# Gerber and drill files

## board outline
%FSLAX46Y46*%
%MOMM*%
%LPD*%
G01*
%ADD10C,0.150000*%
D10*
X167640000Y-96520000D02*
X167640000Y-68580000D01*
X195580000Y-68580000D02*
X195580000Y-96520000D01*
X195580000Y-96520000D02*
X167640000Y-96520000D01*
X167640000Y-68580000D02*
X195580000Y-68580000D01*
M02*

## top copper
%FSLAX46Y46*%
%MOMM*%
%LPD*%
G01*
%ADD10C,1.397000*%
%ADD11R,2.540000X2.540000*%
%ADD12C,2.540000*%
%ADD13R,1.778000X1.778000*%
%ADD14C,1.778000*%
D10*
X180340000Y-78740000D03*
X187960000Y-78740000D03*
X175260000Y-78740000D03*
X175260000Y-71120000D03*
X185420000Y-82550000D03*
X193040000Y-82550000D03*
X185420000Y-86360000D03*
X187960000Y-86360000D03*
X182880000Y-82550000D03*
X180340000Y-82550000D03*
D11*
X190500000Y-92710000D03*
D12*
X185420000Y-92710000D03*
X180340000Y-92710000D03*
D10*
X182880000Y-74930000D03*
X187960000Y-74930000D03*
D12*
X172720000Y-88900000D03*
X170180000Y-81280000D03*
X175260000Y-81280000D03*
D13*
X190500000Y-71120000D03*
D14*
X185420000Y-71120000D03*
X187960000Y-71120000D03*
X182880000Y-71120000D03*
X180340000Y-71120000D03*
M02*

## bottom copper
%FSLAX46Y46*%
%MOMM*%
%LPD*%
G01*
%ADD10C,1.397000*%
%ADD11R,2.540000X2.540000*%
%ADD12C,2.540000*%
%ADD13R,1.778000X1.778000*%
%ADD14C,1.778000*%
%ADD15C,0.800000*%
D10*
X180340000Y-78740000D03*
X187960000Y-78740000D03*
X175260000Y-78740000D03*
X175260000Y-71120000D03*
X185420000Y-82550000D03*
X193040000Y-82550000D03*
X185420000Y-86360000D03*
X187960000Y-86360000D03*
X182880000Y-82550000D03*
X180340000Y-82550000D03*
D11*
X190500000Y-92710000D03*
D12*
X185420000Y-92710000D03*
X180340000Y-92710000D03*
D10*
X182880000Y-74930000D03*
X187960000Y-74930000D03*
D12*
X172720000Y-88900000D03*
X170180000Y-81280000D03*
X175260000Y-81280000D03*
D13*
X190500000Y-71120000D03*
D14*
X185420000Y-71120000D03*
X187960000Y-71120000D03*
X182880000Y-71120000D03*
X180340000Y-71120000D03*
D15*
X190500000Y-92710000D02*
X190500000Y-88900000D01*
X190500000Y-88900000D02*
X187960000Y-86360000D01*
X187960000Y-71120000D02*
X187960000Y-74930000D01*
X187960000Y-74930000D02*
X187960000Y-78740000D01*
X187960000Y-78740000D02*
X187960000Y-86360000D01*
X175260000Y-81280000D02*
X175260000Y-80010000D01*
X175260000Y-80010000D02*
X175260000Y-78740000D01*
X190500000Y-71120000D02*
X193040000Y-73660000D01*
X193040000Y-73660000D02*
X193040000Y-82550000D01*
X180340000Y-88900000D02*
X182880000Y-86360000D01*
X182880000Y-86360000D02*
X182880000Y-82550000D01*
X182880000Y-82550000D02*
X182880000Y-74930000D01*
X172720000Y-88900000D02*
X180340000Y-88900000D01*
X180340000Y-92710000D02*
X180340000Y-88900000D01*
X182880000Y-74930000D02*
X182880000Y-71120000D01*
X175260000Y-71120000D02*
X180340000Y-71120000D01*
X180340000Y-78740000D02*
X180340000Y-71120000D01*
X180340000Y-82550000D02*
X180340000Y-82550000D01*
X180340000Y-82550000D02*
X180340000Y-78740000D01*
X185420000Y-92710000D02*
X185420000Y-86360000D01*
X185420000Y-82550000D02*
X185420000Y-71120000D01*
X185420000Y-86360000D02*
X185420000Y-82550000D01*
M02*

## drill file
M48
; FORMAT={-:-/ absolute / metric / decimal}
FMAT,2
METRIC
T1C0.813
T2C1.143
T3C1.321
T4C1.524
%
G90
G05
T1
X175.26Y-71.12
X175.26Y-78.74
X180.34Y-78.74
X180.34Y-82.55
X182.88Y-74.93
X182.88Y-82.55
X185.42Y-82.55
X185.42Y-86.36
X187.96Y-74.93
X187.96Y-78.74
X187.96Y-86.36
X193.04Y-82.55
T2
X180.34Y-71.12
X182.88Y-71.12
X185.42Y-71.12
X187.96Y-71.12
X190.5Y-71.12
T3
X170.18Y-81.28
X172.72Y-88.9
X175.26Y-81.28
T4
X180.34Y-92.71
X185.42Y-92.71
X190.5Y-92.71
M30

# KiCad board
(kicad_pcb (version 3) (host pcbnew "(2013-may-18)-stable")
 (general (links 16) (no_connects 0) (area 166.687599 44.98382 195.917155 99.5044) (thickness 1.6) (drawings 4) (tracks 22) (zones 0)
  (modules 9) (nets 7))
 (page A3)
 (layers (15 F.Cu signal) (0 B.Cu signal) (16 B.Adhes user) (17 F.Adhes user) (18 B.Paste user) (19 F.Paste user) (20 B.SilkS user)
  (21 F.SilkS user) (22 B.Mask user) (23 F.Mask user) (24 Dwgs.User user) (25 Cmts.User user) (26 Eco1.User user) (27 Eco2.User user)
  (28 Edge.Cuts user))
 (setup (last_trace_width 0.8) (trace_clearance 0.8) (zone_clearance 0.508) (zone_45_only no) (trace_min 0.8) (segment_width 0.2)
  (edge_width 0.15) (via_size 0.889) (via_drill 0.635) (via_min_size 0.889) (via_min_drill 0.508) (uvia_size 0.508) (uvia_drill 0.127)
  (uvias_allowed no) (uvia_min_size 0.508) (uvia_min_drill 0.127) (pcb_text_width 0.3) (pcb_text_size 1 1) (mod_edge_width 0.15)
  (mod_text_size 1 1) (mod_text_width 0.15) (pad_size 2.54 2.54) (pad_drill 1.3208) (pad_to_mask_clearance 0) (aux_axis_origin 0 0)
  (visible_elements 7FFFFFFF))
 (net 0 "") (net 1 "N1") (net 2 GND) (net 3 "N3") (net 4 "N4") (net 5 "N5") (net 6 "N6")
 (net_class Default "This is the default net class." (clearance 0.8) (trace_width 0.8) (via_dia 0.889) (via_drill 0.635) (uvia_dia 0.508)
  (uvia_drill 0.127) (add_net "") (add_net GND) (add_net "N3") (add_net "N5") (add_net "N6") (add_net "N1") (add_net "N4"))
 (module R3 (layer F.Cu) (at 184.15 78.74) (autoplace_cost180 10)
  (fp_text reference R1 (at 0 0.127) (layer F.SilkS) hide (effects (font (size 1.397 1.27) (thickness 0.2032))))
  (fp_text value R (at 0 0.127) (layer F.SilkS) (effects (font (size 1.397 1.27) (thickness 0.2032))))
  (pad 1 thru_hole circle (at -3.81 0) (size 1.397 1.397) (drill 0.8128) (layers *.Cu *.Mask F.SilkS) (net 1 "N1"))
  (pad 2 thru_hole circle (at 3.81 0) (size 1.397 1.397) (drill 0.8128) (layers *.Cu *.Mask F.SilkS) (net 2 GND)))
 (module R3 (layer F.Cu) (at 175.26 74.93 90) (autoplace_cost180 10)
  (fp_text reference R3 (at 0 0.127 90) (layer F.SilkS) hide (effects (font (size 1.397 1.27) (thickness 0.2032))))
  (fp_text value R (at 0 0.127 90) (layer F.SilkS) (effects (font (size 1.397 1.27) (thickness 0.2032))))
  (pad 1 thru_hole circle (at -3.81 0 90) (size 1.397 1.397) (drill 0.8128) (layers *.Cu *.Mask F.SilkS) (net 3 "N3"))
  (pad 2 thru_hole circle (at 3.81 0 90) (size 1.397 1.397) (drill 0.8128) (layers *.Cu *.Mask F.SilkS) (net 1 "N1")))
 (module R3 (layer F.Cu) (at 189.23 82.55) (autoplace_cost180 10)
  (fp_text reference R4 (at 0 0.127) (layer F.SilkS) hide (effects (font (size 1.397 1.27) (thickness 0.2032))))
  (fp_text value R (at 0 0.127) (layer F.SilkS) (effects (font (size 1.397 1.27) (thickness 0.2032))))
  (pad 1 thru_hole circle (at -3.81 0) (size 1.397 1.397) (drill 0.8128) (layers *.Cu *.Mask F.SilkS) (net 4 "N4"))
  (pad 2 thru_hole circle (at 3.81 0) (size 1.397 1.397) (drill 0.8128) (layers *.Cu *.Mask F.SilkS) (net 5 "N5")))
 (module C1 (layer F.Cu) (at 186.69 86.36)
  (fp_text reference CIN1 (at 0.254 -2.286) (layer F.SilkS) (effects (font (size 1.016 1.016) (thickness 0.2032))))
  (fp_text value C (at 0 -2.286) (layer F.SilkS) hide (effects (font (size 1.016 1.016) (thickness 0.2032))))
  (pad 1 thru_hole circle (at -1.27 0) (size 1.397 1.397) (drill 0.8128) (layers *.Cu *.Mask F.SilkS) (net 4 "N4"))
  (pad 2 thru_hole circle (at 1.27 0) (size 1.397 1.397) (drill 0.8128) (layers *.Cu *.Mask F.SilkS) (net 2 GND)))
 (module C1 (layer F.Cu) (at 181.61 82.55 180)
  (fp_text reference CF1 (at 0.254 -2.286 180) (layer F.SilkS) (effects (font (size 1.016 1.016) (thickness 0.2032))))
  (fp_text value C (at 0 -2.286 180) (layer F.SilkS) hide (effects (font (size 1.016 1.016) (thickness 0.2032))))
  (pad 1 thru_hole circle (at -1.27 0 180) (size 1.397 1.397) (drill 0.8128) (layers *.Cu *.Mask F.SilkS) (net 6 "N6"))
  (pad 2 thru_hole circle (at 1.27 0 180) (size 1.397 1.397) (drill 0.8128) (layers *.Cu *.Mask F.SilkS) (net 1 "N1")))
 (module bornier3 (layer F.Cu) (at 185.42 92.71 180)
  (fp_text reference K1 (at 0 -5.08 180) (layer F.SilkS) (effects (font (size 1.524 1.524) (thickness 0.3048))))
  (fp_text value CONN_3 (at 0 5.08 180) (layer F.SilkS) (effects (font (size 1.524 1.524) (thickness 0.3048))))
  (pad 1 thru_hole rect (at -5.08 0 180) (size 2.54 2.54) (drill 1.524) (layers *.Cu *.Mask F.SilkS) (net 2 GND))
  (pad 2 thru_hole circle (at 0 0 180) (size 2.54 2.54) (drill 1.524) (layers *.Cu *.Mask F.SilkS) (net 4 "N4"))
  (pad 3 thru_hole circle (at 5.08 0 180) (size 2.54 2.54) (drill 1.524) (layers *.Cu *.Mask F.SilkS) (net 6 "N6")))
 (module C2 (layer F.Cu) (at 185.42 74.93)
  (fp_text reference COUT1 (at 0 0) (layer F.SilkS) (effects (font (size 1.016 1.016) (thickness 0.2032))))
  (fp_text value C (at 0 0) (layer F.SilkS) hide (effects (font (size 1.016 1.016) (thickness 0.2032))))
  (pad 1 thru_hole circle (at -2.54 0) (size 1.397 1.397) (drill 0.8128) (layers *.Cu *.Mask F.SilkS) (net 6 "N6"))
  (pad 2 thru_hole circle (at 2.54 0) (size 1.397 1.397) (drill 0.8128) (layers *.Cu *.Mask F.SilkS) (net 2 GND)))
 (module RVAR (layer F.Cu) (at 172.72 85.09 180)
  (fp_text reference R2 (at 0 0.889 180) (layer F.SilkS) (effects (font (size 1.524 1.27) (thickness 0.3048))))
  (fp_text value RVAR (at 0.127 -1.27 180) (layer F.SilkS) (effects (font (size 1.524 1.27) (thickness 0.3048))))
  (pad 1 thru_hole circle (at 0 -3.81 180) (size 2.54 2.54) (drill 1.3208) (layers *.Cu *.Mask F.SilkS) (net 6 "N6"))
  (pad 3 thru_hole circle (at 2.54 3.81 180) (size 2.54 2.54) (drill 1.3208) (layers *.Cu *.Mask F.SilkS))
  (pad 2 thru_hole circle (at -2.54 3.81 180) (size 2.54 2.54) (drill 1.3208) (layers *.Cu *.Mask F.SilkS) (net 3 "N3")))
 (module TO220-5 (layer F.Cu) (at 185.42 68.58 90)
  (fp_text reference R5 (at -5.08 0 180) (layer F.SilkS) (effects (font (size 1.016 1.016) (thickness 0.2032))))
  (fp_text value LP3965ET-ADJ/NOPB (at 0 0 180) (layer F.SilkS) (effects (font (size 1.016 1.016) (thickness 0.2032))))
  (pad 1 thru_hole rect (at -2.54 5.08 90) (size 1.778 1.778) (drill 1.143) (layers *.Cu *.Mask F.SilkS) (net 5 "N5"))
  (pad 2 thru_hole circle (at -2.54 0 90) (size 1.778 1.778) (drill 1.143) (layers *.Cu *.Mask F.SilkS) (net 4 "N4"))
  (pad 3 thru_hole circle (at -2.54 2.54 90) (size 1.778 1.778) (drill 1.143) (layers *.Cu *.Mask F.SilkS) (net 2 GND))
  (pad 4 thru_hole circle (at -2.54 -2.54 90) (size 1.778 1.778) (drill 1.143) (layers *.Cu *.Mask F.SilkS) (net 6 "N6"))
  (pad 5 thru_hole circle (at -2.54 -5.08 90) (size 1.778 1.778) (drill 1.143) (layers *.Cu *.Mask F.SilkS) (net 1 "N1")))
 (gr_line (start 167.64 96.52) (end 167.64 68.58) (angle 90) (layer Edge.Cuts) (width 0.15))
 (gr_line (start 195.58 68.58) (end 195.58 96.52) (angle 90) (layer Edge.Cuts) (width 0.15))
 (gr_line (start 195.58 96.52) (end 167.64 96.52) (angle 90) (layer Edge.Cuts) (width 0.15))
 (gr_line (start 167.64 68.58) (end 195.58 68.58) (angle 90) (layer Edge.Cuts) (width 0.15))
 (segment (start 190.5 92.71) (end 190.5 88.9) (width 0.8) (layer B.Cu) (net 2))
 (segment (start 190.5 88.9) (end 187.96 86.36) (width 0.8) (layer B.Cu) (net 2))
 (segment (start 187.96 71.12) (end 187.96 74.93) (width 0.8) (layer B.Cu) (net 2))
 (segment (start 187.96 74.93) (end 187.96 78.74) (width 0.8) (layer B.Cu) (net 2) (status 10))
 (segment (start 187.96 78.74) (end 187.96 86.36) (width 0.8) (layer B.Cu) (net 2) (status 10))
 (segment (start 175.26 81.28) (end 175.26 80.01) (width 0.8) (layer B.Cu) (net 3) (status 10))
 (segment (start 175.26 80.01) (end 175.26 78.74) (width 0.8) (layer B.Cu) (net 3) (status 20))
 (segment (start 190.5 71.12) (end 193.04 73.66) (width 0.8) (layer B.Cu) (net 5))
 (segment (start 193.04 73.66) (end 193.04 82.55) (width 0.8) (layer B.Cu) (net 5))
 (segment (start 180.34 88.9) (end 182.88 86.36) (width 0.8) (layer B.Cu) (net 6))
 (segment (start 182.88 86.36) (end 182.88 82.55) (width 0.8) (layer B.Cu) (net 6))
 (segment (start 182.88 82.55) (end 182.88 74.93) (width 0.8) (layer B.Cu) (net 6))
 (segment (start 172.72 88.9) (end 180.34 88.9) (width 0.8) (layer B.Cu) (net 6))
 (segment (start 180.34 92.71) (end 180.34 88.9) (width 0.8) (layer B.Cu) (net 6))
 (segment (start 182.88 74.93) (end 182.88 71.12) (width 0.8) (layer B.Cu) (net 6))
 (segment (start 175.26 71.12) (end 180.34 71.12) (width 0.8) (layer B.Cu) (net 1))
 (segment (start 180.34 78.74) (end 180.34 71.12) (width 0.8) (layer B.Cu) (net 1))
 (segment (start 180.34 82.55) (end 180.34 82.55) (width 0.8) (layer B.Cu) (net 1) (status 10))
 (segment (start 180.34 82.55) (end 180.34 78.74) (width 0.8) (layer B.Cu) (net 1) (status 10))
 (segment (start 185.42 92.71) (end 185.42 86.36) (width 0.8) (layer B.Cu) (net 4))
 (segment (start 185.42 82.55) (end 185.42 71.12) (width 0.8) (layer B.Cu) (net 4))
 (segment (start 185.42 86.36) (end 185.42 82.55) (width 0.8) (layer B.Cu) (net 4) (status 10)))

